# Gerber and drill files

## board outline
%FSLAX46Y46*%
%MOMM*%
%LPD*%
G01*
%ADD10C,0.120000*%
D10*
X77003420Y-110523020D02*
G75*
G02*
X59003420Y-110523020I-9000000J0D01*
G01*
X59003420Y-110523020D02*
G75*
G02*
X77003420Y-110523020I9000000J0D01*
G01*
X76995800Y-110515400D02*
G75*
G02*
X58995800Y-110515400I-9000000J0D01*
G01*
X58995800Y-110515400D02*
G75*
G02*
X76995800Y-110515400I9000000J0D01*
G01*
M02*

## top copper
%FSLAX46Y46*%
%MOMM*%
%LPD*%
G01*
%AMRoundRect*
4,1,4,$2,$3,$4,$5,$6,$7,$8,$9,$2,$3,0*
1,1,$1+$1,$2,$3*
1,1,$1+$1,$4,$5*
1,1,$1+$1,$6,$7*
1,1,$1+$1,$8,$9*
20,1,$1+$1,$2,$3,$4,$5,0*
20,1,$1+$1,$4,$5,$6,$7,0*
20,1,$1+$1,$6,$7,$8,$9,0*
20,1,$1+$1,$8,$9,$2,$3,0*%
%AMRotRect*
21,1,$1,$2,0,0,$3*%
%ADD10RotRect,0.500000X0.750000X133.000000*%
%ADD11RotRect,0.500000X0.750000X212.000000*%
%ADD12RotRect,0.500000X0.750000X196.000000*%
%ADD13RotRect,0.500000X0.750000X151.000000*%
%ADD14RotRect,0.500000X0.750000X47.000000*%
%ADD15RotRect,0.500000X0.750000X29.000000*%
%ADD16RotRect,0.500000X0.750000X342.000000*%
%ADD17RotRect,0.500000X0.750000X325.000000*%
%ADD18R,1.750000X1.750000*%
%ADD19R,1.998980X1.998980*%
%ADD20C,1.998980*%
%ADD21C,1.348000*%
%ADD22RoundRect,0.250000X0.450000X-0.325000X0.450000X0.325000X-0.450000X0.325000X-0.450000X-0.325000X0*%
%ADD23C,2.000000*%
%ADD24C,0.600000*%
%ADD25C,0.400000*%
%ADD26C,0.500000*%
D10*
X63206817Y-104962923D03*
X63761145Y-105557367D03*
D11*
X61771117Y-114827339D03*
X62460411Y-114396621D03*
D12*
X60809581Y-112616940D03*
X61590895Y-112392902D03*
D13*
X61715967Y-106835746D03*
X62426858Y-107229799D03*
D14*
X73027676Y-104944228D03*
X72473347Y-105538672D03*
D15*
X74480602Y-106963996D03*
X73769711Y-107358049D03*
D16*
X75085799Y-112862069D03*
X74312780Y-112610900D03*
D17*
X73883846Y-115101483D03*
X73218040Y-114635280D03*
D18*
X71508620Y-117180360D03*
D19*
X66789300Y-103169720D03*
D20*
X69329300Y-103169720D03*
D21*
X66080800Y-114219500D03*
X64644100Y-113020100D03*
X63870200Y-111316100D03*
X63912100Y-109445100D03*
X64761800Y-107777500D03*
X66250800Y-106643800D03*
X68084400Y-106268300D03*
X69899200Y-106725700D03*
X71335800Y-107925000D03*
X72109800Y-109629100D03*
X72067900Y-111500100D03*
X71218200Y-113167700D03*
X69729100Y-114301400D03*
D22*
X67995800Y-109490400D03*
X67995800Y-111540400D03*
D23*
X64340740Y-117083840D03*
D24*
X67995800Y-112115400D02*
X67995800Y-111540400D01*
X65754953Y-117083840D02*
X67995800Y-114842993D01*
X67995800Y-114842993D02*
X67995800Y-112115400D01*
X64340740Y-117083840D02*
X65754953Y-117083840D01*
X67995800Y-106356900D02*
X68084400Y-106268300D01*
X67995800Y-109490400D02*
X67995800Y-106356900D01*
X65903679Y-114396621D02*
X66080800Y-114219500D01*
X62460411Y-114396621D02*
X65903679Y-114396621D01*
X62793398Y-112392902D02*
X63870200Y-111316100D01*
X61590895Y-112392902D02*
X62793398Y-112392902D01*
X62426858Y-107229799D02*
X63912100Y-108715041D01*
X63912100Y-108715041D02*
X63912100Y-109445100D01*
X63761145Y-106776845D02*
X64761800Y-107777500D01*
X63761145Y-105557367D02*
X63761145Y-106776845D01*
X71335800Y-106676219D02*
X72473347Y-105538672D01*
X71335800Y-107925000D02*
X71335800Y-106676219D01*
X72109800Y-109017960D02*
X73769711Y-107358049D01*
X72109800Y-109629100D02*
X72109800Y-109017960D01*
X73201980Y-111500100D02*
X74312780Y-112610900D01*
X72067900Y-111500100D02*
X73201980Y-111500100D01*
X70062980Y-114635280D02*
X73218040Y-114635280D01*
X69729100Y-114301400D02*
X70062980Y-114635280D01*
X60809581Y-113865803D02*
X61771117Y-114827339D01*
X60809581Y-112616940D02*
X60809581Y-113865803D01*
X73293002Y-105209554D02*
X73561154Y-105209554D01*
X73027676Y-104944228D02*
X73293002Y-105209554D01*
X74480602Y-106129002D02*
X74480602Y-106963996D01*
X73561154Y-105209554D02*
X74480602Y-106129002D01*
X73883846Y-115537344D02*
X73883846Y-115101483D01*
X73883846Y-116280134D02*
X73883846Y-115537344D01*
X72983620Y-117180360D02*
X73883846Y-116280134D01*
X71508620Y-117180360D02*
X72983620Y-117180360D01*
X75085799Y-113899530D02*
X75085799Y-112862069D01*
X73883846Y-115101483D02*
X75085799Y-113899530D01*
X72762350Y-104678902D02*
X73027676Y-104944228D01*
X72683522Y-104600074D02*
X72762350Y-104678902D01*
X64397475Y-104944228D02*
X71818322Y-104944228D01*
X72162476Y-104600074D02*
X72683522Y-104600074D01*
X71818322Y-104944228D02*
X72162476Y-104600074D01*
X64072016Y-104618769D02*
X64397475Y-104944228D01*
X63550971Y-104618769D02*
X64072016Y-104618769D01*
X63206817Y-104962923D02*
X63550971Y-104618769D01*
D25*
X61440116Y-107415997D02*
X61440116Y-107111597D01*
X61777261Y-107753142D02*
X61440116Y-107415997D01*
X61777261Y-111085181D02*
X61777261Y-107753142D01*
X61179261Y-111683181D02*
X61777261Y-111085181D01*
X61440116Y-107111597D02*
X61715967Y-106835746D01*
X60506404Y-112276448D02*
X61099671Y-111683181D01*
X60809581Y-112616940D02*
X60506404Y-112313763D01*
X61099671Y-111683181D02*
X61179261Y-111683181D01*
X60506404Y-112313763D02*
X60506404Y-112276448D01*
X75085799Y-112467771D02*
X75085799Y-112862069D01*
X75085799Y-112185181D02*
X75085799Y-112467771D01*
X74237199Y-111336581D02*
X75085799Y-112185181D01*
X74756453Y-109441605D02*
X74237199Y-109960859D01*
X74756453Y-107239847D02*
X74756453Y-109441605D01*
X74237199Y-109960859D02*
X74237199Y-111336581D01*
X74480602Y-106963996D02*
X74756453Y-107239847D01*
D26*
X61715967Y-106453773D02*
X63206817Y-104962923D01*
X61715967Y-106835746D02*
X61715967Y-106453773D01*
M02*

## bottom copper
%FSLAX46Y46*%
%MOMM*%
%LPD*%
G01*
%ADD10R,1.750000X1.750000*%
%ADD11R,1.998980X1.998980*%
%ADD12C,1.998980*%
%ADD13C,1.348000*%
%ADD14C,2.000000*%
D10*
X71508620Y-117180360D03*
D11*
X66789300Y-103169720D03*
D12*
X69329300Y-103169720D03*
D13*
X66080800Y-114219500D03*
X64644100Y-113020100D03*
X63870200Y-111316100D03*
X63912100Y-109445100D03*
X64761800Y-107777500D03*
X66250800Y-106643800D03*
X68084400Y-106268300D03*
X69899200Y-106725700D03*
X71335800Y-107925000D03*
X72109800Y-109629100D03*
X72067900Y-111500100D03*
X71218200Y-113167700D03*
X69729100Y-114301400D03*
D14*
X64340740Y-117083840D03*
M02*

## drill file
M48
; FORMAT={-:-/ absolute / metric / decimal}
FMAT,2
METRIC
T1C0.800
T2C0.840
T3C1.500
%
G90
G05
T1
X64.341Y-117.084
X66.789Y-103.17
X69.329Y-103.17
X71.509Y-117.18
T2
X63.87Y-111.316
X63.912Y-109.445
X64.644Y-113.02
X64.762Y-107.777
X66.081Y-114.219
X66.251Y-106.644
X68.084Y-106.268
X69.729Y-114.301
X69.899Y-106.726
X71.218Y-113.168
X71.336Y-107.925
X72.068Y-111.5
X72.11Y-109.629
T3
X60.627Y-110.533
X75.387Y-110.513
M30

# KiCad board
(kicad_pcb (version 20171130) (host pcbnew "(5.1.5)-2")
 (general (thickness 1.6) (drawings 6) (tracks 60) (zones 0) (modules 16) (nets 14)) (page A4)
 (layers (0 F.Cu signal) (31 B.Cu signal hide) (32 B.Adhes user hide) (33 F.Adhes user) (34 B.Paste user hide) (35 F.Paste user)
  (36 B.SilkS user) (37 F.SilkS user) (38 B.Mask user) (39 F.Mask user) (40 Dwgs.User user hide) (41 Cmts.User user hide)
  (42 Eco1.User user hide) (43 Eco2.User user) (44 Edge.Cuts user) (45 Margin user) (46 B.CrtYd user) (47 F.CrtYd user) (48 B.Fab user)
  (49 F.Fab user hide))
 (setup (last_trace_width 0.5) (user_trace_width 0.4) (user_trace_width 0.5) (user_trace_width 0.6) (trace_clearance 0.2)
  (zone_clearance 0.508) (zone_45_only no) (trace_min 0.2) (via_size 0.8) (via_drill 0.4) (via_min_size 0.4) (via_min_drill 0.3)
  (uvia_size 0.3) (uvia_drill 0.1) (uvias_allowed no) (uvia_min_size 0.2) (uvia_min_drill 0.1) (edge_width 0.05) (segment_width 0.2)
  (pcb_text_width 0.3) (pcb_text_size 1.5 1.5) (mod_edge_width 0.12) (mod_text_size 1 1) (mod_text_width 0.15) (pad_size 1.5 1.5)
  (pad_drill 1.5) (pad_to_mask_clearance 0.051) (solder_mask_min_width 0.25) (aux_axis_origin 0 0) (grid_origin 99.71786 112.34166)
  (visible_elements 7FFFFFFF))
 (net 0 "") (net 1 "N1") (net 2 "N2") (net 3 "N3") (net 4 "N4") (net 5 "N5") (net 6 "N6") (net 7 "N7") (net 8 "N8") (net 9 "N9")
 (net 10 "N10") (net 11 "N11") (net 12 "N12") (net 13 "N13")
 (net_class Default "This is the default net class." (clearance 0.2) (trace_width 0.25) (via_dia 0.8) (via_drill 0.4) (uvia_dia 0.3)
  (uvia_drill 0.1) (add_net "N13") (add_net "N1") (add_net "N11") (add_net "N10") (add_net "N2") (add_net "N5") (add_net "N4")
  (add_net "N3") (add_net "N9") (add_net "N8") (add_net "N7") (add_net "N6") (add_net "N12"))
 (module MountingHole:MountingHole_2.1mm (layer F.Cu) (at 75.3872 110.51286)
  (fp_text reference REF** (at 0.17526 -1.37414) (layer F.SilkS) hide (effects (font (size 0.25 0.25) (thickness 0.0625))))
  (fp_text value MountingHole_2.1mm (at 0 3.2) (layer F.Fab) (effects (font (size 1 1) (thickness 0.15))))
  (pad "" np_thru_hole circle (at 0 0) (size 1.5 1.5) (drill 1.5) (layers *.Cu *.Mask)))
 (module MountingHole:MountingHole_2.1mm (layer F.Cu) (at 60.62726 110.53318)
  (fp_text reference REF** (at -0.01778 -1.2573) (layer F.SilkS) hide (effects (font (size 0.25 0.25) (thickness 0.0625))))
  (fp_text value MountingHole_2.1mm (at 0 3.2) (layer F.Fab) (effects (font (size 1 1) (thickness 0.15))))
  (pad "" np_thru_hole circle (at 0 0) (size 1.5 1.5) (drill 1.5) (layers *.Cu *.Mask)))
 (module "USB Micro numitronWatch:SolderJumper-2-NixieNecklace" (layer F.Cu) (at 63.3095 105.11028 133)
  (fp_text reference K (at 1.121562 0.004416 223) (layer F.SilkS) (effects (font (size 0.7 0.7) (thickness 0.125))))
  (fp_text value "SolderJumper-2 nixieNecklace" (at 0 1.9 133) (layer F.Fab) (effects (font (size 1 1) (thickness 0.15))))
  (pad 2 smd rect (at 0.1778 0.0254 133) (size 0.5 0.75) (layers F.Cu F.Mask) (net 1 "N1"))
  (pad 1 smd rect (at -0.635 0.0254 133) (size 0.5 0.75) (layers F.Cu F.Mask) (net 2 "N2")))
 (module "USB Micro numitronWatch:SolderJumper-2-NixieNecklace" (layer F.Cu) (at 61.93536 114.75466 212)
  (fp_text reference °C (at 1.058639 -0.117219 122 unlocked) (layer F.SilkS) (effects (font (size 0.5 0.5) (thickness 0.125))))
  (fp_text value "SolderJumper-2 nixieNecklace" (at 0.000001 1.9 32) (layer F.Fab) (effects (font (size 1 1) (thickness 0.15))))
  (pad 2 smd rect (at 0.1778 0.0254 212) (size 0.5 0.75) (layers F.Cu F.Mask) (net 1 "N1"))
  (pad 1 smd rect (at -0.635 0.0254 212) (size 0.5 0.75) (layers F.Cu F.Mask) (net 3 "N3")))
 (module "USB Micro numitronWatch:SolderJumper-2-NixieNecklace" (layer F.Cu) (at 60.987495 112.592348 196)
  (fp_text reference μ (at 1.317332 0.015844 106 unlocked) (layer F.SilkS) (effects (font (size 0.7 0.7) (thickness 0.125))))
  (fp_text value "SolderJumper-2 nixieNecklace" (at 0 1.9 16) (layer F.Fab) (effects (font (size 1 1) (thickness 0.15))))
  (pad 2 smd rect (at 0.1778 0.0254 196) (size 0.5 0.75) (layers F.Cu F.Mask) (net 1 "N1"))
  (pad 1 smd rect (at -0.635 0.0254 196) (size 0.5 0.75) (layers F.Cu F.Mask) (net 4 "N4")))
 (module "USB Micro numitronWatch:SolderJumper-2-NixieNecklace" (layer F.Cu) (at 61.85916 106.94416 151)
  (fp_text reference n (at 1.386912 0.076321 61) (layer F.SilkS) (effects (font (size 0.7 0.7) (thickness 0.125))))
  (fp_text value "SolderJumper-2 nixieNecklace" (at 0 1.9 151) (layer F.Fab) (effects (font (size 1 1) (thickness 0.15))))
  (pad 2 smd rect (at 0.1778 0.0254 151) (size 0.5 0.75) (layers F.Cu F.Mask) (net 1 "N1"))
  (pad 1 smd rect (at -0.635 0.0254 151) (size 0.5 0.75) (layers F.Cu F.Mask) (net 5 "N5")))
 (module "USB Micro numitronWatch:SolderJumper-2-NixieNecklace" (layer F.Cu) (at 72.88784 105.05694 47)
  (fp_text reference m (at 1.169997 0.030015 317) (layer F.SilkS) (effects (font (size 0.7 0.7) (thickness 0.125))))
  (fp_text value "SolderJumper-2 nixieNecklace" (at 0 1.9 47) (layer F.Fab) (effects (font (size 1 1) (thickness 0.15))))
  (pad 2 smd rect (at 0.1778 0.0254 47) (size 0.5 0.75) (layers F.Cu F.Mask) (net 1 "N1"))
  (pad 1 smd rect (at -0.635 0.0254 47) (size 0.5 0.75) (layers F.Cu F.Mask) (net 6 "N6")))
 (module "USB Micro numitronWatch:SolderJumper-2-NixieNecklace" (layer F.Cu) (at 74.31278 107.02798 29)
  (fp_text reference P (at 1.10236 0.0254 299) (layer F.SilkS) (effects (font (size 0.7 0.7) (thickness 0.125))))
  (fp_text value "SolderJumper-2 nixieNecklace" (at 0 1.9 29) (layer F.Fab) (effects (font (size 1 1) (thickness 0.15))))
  (pad 2 smd rect (at 0.1778 0.0254 29) (size 0.5 0.75) (layers F.Cu F.Mask) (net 1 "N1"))
  (pad 1 smd rect (at -0.635 0.0254 29) (size 0.5 0.75) (layers F.Cu F.Mask) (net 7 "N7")))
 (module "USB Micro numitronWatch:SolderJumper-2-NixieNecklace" (layer F.Cu) (at 74.92455 112.782969 342)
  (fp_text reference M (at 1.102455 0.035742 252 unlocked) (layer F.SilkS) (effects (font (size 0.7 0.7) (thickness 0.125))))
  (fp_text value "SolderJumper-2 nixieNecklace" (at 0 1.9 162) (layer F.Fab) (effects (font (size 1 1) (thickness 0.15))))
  (pad 2 smd rect (at 0.1778 0.0254 342) (size 0.5 0.75) (layers F.Cu F.Mask) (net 1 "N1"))
  (pad 1 smd rect (at -0.635 0.0254 342) (size 0.5 0.75) (layers F.Cu F.Mask) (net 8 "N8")))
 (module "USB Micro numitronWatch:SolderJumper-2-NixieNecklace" (layer F.Cu) (at 73.75277 114.978695 325)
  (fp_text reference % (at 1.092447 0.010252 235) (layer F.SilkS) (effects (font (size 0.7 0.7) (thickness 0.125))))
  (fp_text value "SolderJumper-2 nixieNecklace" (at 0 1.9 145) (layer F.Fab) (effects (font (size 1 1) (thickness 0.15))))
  (pad 2 smd rect (at 0.1778 0.0254 325) (size 0.5 0.75) (layers F.Cu F.Mask) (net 1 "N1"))
  (pad 1 smd rect (at -0.635 0.0254 325) (size 0.5 0.75) (layers F.Cu F.Mask) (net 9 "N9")))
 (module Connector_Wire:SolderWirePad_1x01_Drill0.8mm (layer F.Cu) (at 71.50862 117.18036)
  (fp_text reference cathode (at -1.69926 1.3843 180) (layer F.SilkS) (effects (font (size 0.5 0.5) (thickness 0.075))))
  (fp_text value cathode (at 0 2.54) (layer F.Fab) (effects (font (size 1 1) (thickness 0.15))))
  (pad 1 thru_hole rect (at 0 0) (size 1.75 1.75) (drill 0.8001) (layers *.Cu *.Mask) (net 1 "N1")))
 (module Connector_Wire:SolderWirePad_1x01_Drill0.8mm (layer F.Cu) (at 66.7893 103.16972)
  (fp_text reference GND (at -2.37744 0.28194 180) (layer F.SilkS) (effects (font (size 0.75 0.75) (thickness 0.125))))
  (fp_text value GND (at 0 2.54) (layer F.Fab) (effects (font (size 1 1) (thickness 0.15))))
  (pad 1 thru_hole rect (at 0 0) (size 1.99898 1.99898) (drill 0.8001) (layers *.Cu *.Mask) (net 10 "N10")))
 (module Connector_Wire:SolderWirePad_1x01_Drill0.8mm (layer F.Cu) (at 69.3293 103.16972)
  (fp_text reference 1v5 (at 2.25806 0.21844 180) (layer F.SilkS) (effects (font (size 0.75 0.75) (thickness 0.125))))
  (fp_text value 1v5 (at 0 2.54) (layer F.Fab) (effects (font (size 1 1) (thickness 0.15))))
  (pad 1 thru_hole circle (at 0 0) (size 1.99898 1.99898) (drill 0.8001) (layers *.Cu *.Mask) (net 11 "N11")))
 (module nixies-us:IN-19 (layer F.Cu) (at 67.9958 110.5154)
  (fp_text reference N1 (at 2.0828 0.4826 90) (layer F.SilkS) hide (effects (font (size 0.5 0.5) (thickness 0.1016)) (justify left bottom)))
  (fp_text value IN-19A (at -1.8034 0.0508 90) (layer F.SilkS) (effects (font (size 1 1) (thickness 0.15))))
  (pad 14 thru_hole circle (at -1.915 3.7041 333) (size 1.348 1.348) (drill 0.84) (layers *.Cu *.Mask) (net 3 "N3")
   (solder_mask_margin 0.1016))
  (pad 13 thru_hole circle (at -3.3517 2.5047 333) (size 1.348 1.348) (drill 0.84) (layers *.Cu *.Mask) (solder_mask_margin 0.1016))
  (pad 12 thru_hole circle (at -4.1256 0.8007 333) (size 1.348 1.348) (drill 0.84) (layers *.Cu *.Mask) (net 4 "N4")
   (solder_mask_margin 0.1016))
  (pad 11 thru_hole circle (at -4.0837 -1.0703 333) (size 1.348 1.348) (drill 0.84) (layers *.Cu *.Mask) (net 5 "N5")
   (solder_mask_margin 0.1016))
  (pad 10 thru_hole circle (at -3.234 -2.7379 333) (size 1.348 1.348) (drill 0.84) (layers *.Cu *.Mask) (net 2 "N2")
   (solder_mask_margin 0.1016))
  (pad 9 thru_hole circle (at -1.745 -3.8716 333) (size 1.348 1.348) (drill 0.84) (layers *.Cu *.Mask) (solder_mask_margin 0.1016))
  (pad 8 thru_hole circle (at 0.0886 -4.2471 333) (size 1.348 1.348) (drill 0.84) (layers *.Cu *.Mask) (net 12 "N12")
   (solder_mask_margin 0.1016))
  (pad 7 thru_hole circle (at 1.9034 -3.7897 333) (size 1.348 1.348) (drill 0.84) (layers *.Cu *.Mask) (solder_mask_margin 0.1016))
  (pad 6 thru_hole circle (at 3.34 -2.5904 333) (size 1.348 1.348) (drill 0.84) (layers *.Cu *.Mask) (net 6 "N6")
   (solder_mask_margin 0.1016))
  (pad 5 thru_hole circle (at 4.114 -0.8863 333) (size 1.348 1.348) (drill 0.84) (layers *.Cu *.Mask) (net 7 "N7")
   (solder_mask_margin 0.1016))
  (pad 4 thru_hole circle (at 4.0721 0.9847 333) (size 1.348 1.348) (drill 0.84) (layers *.Cu *.Mask) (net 8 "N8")
   (solder_mask_margin 0.1016))
  (pad 3 thru_hole circle (at 3.2224 2.6523 333) (size 1.348 1.348) (drill 0.84) (layers *.Cu *.Mask) (solder_mask_margin 0.1016))
  (pad 2 thru_hole circle (at 1.7333 3.786 333) (size 1.348 1.348) (drill 0.84) (layers *.Cu *.Mask) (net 9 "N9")
   (solder_mask_margin 0.1016)))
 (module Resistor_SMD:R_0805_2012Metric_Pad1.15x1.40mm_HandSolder (layer F.Cu) (at 67.9958 110.5154 90)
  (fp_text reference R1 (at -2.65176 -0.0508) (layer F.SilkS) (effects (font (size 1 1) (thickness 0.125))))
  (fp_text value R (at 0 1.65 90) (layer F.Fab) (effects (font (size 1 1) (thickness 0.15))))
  (pad 2 smd roundrect (at 1.025 0 90) (size 1.15 1.4) (layers F.Cu F.Paste F.Mask) (roundrect_rratio 0.217391) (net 12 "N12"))
  (pad 1 smd roundrect (at -1.025 0 90) (size 1.15 1.4) (layers F.Cu F.Paste F.Mask) (roundrect_rratio 0.217391) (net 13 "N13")))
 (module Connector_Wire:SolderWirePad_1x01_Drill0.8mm (layer F.Cu) (at 64.34074 117.08384)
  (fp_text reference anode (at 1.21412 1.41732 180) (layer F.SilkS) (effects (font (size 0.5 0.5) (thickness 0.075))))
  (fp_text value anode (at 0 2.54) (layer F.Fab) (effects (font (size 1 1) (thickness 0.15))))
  (pad 1 thru_hole circle (at 0 0) (size 2 2) (drill 0.8001) (layers *.Cu *.Mask) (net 13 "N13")))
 (gr_circle (center 68.00342 110.52302) (end 77.00342 110.52302) (layer Edge.Cuts) (width 0.12))
 (gr_circle (center 67.9958 110.5154) (end 76.9958 110.5154) (layer Edge.Cuts) (width 0.12))
 (segment (start 67.9958 112.1154) (end 67.9958 111.5404) (width 0.6) (layer F.Cu) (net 13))
 (segment (start 65.754953 117.08384) (end 67.9958 114.842993) (width 0.6) (layer F.Cu) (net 13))
 (segment (start 67.9958 114.842993) (end 67.9958 112.1154) (width 0.6) (layer F.Cu) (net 13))
 (segment (start 64.34074 117.08384) (end 65.754953 117.08384) (width 0.6) (layer F.Cu) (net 13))
 (segment (start 67.9958 106.3569) (end 68.0844 106.2683) (width 0.6) (layer F.Cu) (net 12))
 (segment (start 67.9958 109.4904) (end 67.9958 106.3569) (width 0.6) (layer F.Cu) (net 12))
 (segment (start 65.903679 114.396621) (end 66.0808 114.2195) (width 0.6) (layer F.Cu) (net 3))
 (segment (start 62.460411 114.396621) (end 65.903679 114.396621) (width 0.6) (layer F.Cu) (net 3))
 (segment (start 62.793398 112.392902) (end 63.8702 111.3161) (width 0.6) (layer F.Cu) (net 4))
 (segment (start 61.590895 112.392902) (end 62.793398 112.392902) (width 0.6) (layer F.Cu) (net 4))
 (segment (start 62.426858 107.229799) (end 63.9121 108.715041) (width 0.6) (layer F.Cu) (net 5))
 (segment (start 63.9121 108.715041) (end 63.9121 109.4451) (width 0.6) (layer F.Cu) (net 5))
 (segment (start 63.761145 106.776845) (end 64.7618 107.7775) (width 0.6) (layer F.Cu) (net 2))
 (segment (start 63.761145 105.557367) (end 63.761145 106.776845) (width 0.6) (layer F.Cu) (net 2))
 (segment (start 71.3358 106.676219) (end 72.473347 105.538672) (width 0.6) (layer F.Cu) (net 6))
 (segment (start 71.3358 107.925) (end 71.3358 106.676219) (width 0.6) (layer F.Cu) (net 6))
 (segment (start 72.1098 109.01796) (end 73.769711 107.358049) (width 0.6) (layer F.Cu) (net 7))
 (segment (start 72.1098 109.6291) (end 72.1098 109.01796) (width 0.6) (layer F.Cu) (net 7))
 (segment (start 73.20198 111.5001) (end 74.31278 112.6109) (width 0.6) (layer F.Cu) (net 8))
 (segment (start 72.0679 111.5001) (end 73.20198 111.5001) (width 0.6) (layer F.Cu) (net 8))
 (segment (start 70.06298 114.63528) (end 73.21804 114.63528) (width 0.6) (layer F.Cu) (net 9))
 (segment (start 69.7291 114.3014) (end 70.06298 114.63528) (width 0.6) (layer F.Cu) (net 9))
 (segment (start 60.809581 113.865803) (end 61.771117 114.827339) (width 0.6) (layer F.Cu) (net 1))
 (segment (start 60.809581 112.61694) (end 60.809581 113.865803) (width 0.6) (layer F.Cu) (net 1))
 (segment (start 73.293002 105.209554) (end 73.561154 105.209554) (width 0.6) (layer F.Cu) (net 1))
 (segment (start 73.027676 104.944228) (end 73.293002 105.209554) (width 0.6) (layer F.Cu) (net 1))
 (segment (start 74.480602 106.129002) (end 74.480602 106.963996) (width 0.6) (layer F.Cu) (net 1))
 (segment (start 73.561154 105.209554) (end 74.480602 106.129002) (width 0.6) (layer F.Cu) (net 1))
 (segment (start 73.883846 115.537344) (end 73.883846 115.101483) (width 0.6) (layer F.Cu) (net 1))
 (segment (start 73.883846 116.280134) (end 73.883846 115.537344) (width 0.6) (layer F.Cu) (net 1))
 (segment (start 72.98362 117.18036) (end 73.883846 116.280134) (width 0.6) (layer F.Cu) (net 1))
 (segment (start 71.50862 117.18036) (end 72.98362 117.18036) (width 0.6) (layer F.Cu) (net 1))
 (segment (start 75.085799 113.89953) (end 75.085799 112.862069) (width 0.6) (layer F.Cu) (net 1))
 (segment (start 73.883846 115.101483) (end 75.085799 113.89953) (width 0.6) (layer F.Cu) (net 1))
 (segment (start 72.76235 104.678902) (end 73.027676 104.944228) (width 0.6) (layer F.Cu) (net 1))
 (segment (start 72.683522 104.600074) (end 72.76235 104.678902) (width 0.6) (layer F.Cu) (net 1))
 (segment (start 64.397475 104.944228) (end 71.818322 104.944228) (width 0.6) (layer F.Cu) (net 1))
 (segment (start 72.162476 104.600074) (end 72.683522 104.600074) (width 0.6) (layer F.Cu) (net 1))
 (segment (start 71.818322 104.944228) (end 72.162476 104.600074) (width 0.6) (layer F.Cu) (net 1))
 (segment (start 64.072016 104.618769) (end 64.397475 104.944228) (width 0.6) (layer F.Cu) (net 1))
 (segment (start 63.550971 104.618769) (end 64.072016 104.618769) (width 0.6) (layer F.Cu) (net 1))
 (segment (start 63.206817 104.962923) (end 63.550971 104.618769) (width 0.6) (layer F.Cu) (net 1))
 (segment (start 61.440116 107.415997) (end 61.440116 107.111597) (width 0.4) (layer F.Cu) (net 1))
 (segment (start 61.777261 107.753142) (end 61.440116 107.415997) (width 0.4) (layer F.Cu) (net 1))
 (segment (start 61.777261 111.085181) (end 61.777261 107.753142) (width 0.4) (layer F.Cu) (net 1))
 (segment (start 61.179261 111.683181) (end 61.777261 111.085181) (width 0.4) (layer F.Cu) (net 1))
 (segment (start 61.440116 107.111597) (end 61.715967 106.835746) (width 0.4) (layer F.Cu) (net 1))
 (segment (start 60.506404 112.276448) (end 61.099671 111.683181) (width 0.4) (layer F.Cu) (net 1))
 (segment (start 60.809581 112.61694) (end 60.506404 112.313763) (width 0.4) (layer F.Cu) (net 1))
 (segment (start 61.099671 111.683181) (end 61.179261 111.683181) (width 0.4) (layer F.Cu) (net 1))
 (segment (start 60.506404 112.313763) (end 60.506404 112.276448) (width 0.4) (layer F.Cu) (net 1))
 (segment (start 75.085799 112.467771) (end 75.085799 112.862069) (width 0.4) (layer F.Cu) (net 1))
 (segment (start 75.085799 112.185181) (end 75.085799 112.467771) (width 0.4) (layer F.Cu) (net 1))
 (segment (start 74.237199 111.336581) (end 75.085799 112.185181) (width 0.4) (layer F.Cu) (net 1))
 (segment (start 74.756453 109.441605) (end 74.237199 109.960859) (width 0.4) (layer F.Cu) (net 1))
 (segment (start 74.756453 107.239847) (end 74.756453 109.441605) (width 0.4) (layer F.Cu) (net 1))
 (segment (start 74.237199 109.960859) (end 74.237199 111.336581) (width 0.4) (layer F.Cu) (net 1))
 (segment (start 74.480602 106.963996) (end 74.756453 107.239847) (width 0.4) (layer F.Cu) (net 1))
 (segment (start 61.715967 106.453773) (end 63.206817 104.962923) (width 0.5) (layer F.Cu) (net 1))
 (segment (start 61.715967 106.835746) (end 61.715967 106.453773) (width 0.5) (layer F.Cu) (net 1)))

